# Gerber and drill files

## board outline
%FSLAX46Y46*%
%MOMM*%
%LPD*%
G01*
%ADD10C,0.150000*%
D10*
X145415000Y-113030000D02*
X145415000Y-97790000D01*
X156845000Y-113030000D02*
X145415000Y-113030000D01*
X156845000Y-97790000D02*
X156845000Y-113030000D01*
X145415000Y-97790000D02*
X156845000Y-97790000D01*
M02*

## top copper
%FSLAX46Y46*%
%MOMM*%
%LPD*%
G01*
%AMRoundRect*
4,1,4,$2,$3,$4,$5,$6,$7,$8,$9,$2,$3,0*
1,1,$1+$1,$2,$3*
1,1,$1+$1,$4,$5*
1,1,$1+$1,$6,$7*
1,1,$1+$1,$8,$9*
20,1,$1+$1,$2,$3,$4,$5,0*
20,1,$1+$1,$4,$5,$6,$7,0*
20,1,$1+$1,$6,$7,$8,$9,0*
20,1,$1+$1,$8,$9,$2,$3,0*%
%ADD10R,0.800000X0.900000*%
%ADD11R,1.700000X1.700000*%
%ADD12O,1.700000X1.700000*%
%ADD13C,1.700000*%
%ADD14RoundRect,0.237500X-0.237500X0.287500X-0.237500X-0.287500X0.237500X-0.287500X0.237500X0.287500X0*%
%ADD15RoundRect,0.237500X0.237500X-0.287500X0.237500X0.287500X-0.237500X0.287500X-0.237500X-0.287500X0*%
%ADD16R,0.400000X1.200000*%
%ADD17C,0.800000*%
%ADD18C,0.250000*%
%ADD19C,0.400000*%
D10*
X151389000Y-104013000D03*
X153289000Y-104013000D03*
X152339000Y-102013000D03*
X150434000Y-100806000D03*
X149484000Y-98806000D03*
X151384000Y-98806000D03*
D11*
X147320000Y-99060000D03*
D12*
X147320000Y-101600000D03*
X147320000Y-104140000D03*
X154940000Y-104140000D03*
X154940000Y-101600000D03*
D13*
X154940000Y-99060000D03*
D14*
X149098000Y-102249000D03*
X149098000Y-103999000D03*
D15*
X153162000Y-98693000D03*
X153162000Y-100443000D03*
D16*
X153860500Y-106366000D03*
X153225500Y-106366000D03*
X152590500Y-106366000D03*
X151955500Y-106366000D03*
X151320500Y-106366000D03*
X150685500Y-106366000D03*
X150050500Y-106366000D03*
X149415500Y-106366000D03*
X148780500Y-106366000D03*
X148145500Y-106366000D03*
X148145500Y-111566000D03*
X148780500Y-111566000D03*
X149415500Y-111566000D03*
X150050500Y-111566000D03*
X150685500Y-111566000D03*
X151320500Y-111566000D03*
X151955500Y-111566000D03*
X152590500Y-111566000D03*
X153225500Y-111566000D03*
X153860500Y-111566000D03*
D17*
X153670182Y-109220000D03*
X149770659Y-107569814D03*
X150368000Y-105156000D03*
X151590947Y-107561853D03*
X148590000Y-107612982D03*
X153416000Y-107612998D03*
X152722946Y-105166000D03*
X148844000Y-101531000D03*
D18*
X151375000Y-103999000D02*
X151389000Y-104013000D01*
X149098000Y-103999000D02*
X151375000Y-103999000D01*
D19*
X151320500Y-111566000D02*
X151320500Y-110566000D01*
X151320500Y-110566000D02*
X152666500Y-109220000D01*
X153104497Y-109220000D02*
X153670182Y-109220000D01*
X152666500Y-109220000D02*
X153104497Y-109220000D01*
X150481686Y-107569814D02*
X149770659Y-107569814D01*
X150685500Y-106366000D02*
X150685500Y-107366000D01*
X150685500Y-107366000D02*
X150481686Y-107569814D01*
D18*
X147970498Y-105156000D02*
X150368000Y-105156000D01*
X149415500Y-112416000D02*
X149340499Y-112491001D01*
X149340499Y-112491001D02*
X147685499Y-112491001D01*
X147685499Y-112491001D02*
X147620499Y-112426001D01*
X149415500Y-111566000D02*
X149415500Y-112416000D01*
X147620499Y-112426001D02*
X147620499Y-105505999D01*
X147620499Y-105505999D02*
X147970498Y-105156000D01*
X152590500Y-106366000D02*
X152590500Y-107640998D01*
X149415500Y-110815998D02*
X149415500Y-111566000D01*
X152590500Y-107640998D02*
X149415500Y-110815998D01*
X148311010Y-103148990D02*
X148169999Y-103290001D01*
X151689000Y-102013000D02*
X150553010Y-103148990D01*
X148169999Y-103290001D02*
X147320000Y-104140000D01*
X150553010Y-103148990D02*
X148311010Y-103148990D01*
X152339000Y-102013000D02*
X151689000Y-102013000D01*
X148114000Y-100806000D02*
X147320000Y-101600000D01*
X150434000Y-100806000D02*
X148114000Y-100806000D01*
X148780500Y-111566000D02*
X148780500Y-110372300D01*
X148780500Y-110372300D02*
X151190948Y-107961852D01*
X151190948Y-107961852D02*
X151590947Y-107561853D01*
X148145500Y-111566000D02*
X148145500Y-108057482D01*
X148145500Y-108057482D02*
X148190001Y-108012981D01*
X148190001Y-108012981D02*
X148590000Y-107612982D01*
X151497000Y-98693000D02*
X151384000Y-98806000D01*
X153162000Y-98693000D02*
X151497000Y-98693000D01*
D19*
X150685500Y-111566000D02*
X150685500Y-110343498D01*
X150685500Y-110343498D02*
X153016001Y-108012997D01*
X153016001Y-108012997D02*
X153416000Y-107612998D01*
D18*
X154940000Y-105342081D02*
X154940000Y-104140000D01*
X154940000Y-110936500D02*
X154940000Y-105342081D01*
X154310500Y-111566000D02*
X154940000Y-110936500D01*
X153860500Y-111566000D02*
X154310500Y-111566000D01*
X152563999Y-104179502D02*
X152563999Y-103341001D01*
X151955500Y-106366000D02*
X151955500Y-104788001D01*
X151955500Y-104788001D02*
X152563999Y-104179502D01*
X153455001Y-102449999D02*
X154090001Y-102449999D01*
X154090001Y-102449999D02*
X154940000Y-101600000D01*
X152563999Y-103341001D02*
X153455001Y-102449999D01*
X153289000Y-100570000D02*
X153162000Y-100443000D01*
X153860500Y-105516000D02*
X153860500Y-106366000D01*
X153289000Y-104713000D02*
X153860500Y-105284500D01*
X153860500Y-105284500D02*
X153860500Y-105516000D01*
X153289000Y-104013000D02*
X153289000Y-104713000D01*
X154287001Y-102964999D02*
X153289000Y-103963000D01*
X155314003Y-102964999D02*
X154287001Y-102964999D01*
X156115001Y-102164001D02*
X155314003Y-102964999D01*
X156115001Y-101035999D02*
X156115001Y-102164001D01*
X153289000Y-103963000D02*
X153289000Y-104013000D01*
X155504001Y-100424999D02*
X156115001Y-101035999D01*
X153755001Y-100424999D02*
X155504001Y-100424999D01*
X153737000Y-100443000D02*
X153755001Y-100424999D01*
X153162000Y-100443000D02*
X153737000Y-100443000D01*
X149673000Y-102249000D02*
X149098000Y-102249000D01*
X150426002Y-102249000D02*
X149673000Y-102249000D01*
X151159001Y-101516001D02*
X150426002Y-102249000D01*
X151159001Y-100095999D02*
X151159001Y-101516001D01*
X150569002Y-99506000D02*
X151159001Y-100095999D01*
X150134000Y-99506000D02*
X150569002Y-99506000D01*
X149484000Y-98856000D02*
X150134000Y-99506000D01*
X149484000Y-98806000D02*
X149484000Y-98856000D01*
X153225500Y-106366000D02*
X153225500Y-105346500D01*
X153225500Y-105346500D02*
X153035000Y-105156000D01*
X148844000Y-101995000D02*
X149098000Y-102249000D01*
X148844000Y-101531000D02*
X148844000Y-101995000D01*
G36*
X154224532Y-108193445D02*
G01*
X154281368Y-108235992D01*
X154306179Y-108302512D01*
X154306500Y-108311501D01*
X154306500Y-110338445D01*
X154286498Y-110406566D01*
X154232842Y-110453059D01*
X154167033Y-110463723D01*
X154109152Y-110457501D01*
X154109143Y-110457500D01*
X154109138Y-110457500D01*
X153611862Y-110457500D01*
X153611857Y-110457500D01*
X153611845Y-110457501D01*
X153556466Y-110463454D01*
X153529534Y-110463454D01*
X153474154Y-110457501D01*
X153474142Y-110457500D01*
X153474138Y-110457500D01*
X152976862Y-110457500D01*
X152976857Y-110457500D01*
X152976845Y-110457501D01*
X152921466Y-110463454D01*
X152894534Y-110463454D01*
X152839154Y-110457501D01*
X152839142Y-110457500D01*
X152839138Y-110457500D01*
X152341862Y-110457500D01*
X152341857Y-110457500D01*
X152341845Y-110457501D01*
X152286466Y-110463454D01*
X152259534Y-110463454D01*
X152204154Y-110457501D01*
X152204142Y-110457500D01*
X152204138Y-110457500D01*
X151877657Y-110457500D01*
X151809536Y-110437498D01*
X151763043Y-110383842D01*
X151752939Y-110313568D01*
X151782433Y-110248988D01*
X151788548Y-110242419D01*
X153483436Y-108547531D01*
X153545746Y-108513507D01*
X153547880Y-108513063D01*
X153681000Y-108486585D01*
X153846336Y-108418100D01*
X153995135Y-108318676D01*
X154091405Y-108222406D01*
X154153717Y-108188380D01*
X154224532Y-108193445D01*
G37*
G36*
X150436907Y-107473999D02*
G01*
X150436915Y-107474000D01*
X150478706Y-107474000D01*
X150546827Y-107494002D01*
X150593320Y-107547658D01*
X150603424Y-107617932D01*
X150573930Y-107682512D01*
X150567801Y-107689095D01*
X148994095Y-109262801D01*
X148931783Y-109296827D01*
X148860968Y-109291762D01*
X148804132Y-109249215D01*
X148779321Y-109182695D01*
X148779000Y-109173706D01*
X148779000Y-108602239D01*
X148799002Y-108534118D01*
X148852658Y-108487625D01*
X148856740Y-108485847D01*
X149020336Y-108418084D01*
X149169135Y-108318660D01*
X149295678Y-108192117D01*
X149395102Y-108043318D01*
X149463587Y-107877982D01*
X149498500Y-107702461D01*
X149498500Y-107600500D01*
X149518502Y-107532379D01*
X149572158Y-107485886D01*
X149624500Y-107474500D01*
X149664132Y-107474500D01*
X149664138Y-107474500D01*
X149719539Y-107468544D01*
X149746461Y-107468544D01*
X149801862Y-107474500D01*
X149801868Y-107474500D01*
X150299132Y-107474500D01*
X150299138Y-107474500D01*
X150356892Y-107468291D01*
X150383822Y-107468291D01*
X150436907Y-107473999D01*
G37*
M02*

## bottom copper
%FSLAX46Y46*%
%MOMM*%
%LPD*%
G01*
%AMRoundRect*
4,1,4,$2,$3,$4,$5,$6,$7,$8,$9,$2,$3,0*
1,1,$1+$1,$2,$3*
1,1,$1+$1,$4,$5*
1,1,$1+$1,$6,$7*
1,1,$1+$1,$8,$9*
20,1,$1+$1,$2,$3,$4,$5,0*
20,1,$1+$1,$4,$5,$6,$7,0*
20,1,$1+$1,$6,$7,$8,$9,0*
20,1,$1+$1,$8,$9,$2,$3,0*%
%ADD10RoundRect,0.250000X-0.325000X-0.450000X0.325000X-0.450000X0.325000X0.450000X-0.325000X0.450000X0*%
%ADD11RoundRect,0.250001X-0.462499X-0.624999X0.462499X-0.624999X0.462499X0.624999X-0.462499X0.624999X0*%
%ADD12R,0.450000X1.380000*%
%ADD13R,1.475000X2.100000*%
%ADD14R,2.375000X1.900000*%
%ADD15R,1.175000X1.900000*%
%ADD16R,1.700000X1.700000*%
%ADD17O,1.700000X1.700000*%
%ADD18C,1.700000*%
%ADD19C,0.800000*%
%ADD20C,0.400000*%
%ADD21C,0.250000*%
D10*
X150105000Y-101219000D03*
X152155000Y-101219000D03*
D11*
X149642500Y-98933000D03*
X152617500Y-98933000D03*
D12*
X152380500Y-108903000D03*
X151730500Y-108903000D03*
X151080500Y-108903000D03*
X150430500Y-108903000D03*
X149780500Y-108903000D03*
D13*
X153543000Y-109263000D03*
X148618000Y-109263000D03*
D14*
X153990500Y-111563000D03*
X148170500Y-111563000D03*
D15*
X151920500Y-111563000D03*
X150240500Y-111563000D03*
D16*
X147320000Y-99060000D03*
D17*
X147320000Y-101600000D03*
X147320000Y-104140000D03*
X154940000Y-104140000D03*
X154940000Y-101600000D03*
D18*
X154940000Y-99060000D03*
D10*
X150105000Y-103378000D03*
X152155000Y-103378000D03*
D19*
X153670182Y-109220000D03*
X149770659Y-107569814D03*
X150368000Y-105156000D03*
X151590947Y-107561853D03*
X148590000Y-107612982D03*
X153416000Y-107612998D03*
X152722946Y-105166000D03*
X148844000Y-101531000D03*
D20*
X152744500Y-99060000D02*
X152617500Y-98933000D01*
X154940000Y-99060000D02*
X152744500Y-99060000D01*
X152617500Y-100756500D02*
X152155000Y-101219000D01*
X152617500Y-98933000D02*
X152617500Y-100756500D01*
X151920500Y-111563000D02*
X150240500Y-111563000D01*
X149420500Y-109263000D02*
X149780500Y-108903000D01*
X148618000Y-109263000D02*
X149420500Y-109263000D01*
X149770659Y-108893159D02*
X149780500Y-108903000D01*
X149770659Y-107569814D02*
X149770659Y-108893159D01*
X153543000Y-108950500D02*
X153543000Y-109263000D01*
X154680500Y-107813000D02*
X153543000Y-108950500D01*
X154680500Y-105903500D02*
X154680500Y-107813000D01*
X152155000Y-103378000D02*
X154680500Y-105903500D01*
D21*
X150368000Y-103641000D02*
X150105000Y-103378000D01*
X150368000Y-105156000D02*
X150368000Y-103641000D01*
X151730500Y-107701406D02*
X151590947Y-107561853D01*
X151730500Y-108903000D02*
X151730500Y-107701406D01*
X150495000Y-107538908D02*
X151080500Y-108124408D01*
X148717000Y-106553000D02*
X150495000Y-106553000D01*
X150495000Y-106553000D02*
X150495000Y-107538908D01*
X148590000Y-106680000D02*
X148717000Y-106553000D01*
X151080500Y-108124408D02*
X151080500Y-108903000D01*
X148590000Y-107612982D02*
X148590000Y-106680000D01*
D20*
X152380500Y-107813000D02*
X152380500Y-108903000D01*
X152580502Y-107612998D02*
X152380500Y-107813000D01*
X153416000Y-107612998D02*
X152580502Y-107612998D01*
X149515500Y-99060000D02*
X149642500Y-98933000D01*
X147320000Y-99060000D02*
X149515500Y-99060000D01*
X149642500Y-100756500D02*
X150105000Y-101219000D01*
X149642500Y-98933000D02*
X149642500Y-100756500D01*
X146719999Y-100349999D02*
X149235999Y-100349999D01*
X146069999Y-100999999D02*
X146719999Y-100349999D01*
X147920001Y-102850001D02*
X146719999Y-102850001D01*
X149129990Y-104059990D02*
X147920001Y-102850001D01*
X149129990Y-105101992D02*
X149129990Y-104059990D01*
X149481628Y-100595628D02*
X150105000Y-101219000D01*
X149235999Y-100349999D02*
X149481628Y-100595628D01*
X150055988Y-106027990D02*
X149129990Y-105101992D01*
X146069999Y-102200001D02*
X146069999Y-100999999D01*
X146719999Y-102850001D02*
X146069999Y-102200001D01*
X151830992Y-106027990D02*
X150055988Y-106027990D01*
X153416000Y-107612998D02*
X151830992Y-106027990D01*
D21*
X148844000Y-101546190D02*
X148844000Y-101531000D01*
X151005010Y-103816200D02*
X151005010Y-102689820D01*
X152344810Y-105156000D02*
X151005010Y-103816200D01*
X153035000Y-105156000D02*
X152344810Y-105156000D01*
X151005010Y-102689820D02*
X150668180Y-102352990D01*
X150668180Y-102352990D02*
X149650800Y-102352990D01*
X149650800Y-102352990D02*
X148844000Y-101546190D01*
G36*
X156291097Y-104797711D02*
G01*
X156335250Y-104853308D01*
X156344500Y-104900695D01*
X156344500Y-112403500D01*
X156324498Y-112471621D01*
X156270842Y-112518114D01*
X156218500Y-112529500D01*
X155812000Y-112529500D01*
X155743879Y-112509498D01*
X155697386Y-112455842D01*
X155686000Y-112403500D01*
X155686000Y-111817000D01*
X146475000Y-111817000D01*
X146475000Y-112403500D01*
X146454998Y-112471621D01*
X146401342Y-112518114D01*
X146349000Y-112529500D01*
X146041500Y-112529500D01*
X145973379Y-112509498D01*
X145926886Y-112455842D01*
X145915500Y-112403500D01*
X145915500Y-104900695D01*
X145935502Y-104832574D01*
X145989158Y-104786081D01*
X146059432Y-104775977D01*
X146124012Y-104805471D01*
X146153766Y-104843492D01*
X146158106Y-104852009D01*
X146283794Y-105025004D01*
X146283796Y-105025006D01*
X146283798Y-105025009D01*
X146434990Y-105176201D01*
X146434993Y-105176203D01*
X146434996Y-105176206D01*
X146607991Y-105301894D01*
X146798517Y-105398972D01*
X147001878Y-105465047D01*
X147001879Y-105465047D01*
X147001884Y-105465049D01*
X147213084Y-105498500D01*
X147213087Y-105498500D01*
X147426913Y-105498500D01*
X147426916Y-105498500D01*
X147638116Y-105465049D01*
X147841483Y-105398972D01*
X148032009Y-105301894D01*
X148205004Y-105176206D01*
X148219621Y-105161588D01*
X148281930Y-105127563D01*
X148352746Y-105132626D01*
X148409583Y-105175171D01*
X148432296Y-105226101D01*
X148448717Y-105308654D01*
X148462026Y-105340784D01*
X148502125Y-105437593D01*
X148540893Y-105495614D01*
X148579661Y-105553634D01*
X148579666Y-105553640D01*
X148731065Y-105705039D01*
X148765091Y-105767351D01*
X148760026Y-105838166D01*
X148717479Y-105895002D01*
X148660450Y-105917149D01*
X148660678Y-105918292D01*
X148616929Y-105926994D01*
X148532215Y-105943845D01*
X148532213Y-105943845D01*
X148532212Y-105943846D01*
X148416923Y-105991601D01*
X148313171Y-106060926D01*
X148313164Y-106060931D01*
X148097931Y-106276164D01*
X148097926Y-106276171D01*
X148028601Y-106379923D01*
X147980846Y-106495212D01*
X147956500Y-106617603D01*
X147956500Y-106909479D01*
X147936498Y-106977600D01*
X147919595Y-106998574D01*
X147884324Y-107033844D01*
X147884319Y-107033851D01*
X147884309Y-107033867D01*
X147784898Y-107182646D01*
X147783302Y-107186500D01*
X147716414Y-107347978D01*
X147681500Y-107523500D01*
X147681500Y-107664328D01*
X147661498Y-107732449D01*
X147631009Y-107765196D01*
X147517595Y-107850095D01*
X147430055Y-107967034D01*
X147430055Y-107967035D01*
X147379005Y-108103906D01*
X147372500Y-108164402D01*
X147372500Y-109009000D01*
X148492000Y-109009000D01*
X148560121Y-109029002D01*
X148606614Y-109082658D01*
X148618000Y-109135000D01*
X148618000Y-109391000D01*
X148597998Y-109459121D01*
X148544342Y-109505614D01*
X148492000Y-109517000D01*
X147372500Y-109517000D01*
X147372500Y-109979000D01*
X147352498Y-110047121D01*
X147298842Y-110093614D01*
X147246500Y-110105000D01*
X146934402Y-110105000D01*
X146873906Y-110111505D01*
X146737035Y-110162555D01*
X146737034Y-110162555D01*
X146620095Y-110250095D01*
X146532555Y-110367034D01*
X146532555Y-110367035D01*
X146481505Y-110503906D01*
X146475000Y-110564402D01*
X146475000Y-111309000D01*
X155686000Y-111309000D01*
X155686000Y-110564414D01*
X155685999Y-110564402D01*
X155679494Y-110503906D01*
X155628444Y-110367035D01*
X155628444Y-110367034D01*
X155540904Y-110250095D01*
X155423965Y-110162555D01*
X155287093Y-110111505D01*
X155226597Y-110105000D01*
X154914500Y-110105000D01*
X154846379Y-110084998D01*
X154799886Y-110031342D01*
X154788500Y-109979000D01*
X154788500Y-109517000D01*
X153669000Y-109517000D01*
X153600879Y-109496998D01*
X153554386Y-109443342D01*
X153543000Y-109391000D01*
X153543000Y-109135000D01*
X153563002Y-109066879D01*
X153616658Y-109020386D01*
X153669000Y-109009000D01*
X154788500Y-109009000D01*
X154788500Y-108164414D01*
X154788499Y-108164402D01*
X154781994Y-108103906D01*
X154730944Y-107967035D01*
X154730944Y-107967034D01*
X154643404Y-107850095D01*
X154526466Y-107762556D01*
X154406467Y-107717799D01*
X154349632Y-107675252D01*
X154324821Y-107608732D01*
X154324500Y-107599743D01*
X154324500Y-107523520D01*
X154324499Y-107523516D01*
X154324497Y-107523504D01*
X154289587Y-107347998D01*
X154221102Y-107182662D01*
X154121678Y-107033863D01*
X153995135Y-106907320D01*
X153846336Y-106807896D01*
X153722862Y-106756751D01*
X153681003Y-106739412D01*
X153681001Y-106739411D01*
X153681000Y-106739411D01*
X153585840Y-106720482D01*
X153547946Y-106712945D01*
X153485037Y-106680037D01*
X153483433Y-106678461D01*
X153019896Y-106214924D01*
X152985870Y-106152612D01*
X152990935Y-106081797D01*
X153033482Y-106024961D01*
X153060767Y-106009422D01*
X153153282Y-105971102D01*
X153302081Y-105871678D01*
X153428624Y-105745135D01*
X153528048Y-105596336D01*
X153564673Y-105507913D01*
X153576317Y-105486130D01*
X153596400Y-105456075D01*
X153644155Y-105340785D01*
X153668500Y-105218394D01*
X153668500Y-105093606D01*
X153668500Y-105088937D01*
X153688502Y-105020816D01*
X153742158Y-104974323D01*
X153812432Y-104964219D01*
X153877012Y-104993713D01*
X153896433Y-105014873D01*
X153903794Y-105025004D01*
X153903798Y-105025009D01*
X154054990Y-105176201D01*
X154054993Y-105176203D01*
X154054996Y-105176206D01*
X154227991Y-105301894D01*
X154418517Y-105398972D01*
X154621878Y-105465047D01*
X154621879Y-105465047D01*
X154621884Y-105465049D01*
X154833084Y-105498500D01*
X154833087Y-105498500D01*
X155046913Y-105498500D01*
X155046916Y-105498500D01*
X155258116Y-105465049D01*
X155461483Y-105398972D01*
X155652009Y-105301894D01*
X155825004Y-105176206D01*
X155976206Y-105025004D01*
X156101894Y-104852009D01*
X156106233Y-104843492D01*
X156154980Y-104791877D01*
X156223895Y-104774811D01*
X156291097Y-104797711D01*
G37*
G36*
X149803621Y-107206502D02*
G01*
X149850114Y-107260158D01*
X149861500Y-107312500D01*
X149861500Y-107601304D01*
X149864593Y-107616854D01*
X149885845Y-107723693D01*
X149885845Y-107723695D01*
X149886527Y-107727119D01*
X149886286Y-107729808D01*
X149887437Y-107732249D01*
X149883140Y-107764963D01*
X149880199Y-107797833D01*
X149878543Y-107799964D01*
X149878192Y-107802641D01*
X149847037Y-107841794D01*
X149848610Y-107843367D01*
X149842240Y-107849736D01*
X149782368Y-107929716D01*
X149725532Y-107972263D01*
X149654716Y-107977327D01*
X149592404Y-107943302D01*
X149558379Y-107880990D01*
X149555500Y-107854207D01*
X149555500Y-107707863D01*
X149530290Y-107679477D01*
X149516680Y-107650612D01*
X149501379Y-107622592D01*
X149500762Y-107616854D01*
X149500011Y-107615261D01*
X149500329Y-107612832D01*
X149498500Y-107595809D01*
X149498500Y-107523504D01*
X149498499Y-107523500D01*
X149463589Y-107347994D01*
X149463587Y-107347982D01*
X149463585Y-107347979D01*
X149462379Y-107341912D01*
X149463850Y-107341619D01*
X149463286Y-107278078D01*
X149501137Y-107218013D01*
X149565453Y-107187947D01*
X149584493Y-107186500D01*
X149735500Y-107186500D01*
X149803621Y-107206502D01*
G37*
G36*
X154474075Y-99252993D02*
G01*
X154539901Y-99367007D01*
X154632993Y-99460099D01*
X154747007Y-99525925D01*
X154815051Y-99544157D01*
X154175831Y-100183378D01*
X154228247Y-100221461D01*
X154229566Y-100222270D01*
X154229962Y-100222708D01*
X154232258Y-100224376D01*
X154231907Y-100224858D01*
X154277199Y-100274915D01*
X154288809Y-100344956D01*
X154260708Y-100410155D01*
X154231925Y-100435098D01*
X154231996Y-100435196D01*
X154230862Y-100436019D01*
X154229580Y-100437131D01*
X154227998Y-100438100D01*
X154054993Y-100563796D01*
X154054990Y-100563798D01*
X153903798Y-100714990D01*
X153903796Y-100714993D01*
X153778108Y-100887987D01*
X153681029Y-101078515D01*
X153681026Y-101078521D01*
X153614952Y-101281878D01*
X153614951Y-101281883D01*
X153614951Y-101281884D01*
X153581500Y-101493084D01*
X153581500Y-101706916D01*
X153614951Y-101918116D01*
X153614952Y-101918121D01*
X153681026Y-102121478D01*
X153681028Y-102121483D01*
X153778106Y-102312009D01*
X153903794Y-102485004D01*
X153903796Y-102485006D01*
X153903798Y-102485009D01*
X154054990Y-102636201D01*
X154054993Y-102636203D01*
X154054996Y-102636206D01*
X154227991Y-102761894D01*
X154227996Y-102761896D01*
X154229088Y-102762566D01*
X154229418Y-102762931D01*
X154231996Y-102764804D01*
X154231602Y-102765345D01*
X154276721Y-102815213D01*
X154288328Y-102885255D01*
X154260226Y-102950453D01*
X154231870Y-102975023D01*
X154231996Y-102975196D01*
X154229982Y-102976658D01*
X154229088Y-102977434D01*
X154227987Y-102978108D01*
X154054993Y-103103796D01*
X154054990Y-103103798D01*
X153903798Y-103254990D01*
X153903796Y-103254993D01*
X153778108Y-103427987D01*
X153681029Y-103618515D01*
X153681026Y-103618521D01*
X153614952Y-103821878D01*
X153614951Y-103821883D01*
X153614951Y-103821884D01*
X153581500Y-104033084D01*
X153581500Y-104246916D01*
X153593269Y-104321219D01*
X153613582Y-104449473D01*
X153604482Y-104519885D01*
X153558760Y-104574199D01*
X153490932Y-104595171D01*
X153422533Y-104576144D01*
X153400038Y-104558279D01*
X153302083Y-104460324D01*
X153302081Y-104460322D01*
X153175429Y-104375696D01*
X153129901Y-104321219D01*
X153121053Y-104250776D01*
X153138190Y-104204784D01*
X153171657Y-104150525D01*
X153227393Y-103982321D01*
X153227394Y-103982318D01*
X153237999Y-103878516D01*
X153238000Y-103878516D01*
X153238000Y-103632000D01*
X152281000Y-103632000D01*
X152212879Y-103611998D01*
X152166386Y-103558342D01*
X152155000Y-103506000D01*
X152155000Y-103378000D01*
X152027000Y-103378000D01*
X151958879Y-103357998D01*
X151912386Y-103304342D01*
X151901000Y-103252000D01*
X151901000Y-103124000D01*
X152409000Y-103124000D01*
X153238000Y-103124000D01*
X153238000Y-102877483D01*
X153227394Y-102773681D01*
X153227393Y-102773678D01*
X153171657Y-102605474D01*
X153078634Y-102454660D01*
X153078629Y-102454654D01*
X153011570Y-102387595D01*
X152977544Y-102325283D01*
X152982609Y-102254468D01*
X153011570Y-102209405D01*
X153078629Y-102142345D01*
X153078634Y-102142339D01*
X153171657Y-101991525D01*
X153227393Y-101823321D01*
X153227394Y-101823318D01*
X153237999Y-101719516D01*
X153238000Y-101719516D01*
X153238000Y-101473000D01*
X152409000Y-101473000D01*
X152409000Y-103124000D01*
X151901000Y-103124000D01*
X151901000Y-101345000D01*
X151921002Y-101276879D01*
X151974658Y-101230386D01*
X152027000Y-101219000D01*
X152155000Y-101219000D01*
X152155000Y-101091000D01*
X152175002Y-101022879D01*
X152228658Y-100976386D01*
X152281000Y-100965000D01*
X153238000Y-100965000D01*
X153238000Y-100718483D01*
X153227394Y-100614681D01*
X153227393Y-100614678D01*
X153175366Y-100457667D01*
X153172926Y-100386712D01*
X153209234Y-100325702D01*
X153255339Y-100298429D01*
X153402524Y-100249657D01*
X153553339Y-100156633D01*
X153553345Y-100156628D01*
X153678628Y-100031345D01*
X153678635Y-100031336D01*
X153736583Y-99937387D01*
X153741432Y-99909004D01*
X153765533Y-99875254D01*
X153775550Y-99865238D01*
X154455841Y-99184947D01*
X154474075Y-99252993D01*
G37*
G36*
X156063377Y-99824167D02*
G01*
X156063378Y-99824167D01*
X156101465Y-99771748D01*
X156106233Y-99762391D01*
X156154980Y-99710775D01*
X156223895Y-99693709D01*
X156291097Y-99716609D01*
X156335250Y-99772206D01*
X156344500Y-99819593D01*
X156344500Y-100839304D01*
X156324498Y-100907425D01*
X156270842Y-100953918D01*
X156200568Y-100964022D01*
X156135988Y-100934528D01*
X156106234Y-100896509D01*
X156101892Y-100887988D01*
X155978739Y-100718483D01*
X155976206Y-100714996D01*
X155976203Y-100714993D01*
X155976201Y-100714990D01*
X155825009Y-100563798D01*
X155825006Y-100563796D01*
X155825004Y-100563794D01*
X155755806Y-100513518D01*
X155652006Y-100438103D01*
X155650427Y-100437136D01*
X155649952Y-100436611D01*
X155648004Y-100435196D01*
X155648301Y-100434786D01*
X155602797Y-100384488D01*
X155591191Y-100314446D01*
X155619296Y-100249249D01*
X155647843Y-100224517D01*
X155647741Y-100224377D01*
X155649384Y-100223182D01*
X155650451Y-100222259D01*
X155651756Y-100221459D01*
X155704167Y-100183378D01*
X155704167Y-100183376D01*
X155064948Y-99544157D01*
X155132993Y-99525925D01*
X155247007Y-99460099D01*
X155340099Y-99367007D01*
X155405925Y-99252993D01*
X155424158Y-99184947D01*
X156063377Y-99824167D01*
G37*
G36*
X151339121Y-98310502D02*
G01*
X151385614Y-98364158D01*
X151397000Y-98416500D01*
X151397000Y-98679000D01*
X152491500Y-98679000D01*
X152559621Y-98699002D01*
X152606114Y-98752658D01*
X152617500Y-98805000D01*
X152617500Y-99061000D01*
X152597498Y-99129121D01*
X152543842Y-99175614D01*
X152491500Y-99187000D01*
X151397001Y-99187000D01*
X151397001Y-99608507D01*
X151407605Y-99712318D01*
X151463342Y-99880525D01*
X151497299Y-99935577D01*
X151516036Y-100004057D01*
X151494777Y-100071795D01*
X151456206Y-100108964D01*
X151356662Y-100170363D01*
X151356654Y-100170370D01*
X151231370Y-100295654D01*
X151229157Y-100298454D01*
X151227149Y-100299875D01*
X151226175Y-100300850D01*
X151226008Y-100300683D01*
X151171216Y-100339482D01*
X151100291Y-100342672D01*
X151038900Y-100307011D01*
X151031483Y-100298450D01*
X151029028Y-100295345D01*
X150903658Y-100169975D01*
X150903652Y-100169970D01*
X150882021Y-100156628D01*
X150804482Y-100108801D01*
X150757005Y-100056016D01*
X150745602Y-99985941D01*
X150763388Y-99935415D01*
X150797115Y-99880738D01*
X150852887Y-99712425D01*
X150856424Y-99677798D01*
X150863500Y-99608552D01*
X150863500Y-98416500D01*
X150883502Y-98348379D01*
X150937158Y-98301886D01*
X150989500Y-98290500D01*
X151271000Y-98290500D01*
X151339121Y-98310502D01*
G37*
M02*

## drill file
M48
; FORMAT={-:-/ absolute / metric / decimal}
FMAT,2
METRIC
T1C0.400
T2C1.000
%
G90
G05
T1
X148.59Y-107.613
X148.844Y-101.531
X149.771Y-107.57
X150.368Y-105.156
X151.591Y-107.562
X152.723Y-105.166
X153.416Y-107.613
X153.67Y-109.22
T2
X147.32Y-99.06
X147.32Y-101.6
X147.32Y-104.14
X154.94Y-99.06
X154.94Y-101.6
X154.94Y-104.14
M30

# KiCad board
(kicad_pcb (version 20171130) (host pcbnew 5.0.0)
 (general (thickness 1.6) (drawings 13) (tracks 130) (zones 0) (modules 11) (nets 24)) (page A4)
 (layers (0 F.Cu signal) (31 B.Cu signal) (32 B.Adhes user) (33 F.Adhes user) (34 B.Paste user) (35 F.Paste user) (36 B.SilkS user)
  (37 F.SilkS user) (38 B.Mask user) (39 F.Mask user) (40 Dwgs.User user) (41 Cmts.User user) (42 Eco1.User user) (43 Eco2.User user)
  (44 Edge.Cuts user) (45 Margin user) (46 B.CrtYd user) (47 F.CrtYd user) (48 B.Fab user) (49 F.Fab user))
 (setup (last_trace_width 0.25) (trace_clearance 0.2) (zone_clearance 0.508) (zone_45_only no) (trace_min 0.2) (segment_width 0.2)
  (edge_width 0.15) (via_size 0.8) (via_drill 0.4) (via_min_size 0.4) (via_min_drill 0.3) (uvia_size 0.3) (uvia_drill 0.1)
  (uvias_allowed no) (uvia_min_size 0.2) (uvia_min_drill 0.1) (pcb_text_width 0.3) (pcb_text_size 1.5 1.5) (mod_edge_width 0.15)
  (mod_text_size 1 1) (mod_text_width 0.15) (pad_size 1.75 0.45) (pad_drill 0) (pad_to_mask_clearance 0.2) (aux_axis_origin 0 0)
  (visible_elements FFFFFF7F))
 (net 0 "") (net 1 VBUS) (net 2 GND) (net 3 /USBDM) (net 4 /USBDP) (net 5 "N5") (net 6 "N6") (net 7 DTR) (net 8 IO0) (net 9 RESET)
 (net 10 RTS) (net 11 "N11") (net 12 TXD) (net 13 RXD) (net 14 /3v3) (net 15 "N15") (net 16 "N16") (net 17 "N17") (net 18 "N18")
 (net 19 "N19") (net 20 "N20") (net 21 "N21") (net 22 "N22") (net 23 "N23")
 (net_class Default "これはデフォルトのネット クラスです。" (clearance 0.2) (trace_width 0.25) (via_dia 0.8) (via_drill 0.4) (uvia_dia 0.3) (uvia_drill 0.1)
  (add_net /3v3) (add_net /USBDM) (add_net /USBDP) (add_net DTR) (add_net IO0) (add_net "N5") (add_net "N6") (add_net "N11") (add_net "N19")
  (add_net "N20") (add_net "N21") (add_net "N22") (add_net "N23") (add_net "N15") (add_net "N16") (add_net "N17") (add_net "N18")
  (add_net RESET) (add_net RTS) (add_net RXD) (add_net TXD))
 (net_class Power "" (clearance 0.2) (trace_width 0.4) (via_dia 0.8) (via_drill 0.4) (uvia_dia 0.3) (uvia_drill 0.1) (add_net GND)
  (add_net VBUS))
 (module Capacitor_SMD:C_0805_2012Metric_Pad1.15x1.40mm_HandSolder (layer B.Cu) (at 151.13 101.219)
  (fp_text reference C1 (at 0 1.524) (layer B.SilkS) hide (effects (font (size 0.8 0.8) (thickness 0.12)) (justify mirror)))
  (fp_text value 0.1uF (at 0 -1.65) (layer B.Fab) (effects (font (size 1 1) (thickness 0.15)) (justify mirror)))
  (pad 1 smd roundrect (at -1.025 0) (size 1.15 1.4) (layers B.Cu B.Paste B.Mask) (roundrect_rratio 0.217391) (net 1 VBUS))
  (pad 2 smd roundrect (at 1.025 0) (size 1.15 1.4) (layers B.Cu B.Paste B.Mask) (roundrect_rratio 0.217391) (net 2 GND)))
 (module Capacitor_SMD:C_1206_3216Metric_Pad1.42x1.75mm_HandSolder (layer B.Cu) (at 151.13 98.933)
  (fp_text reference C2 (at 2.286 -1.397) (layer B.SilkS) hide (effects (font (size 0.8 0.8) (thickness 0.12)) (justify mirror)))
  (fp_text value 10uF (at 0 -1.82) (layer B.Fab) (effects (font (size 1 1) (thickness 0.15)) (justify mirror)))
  (pad 1 smd roundrect (at -1.4875 0) (size 1.425 1.75) (layers B.Cu B.Paste B.Mask) (roundrect_rratio 0.175439) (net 1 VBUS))
  (pad 2 smd roundrect (at 1.4875 0) (size 1.425 1.75) (layers B.Cu B.Paste B.Mask) (roundrect_rratio 0.175439) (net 2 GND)))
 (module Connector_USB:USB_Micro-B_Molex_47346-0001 (layer B.Cu) (at 151.0805 110.363 180)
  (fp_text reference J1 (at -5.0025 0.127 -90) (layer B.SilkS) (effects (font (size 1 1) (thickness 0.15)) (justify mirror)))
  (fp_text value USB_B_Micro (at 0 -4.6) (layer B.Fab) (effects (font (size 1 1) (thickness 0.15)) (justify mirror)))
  (pad 1 smd rect (at -1.3 1.46 180) (size 0.45 1.38) (layers B.Cu B.Paste B.Mask) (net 1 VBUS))
  (pad 2 smd rect (at -0.65 1.46 180) (size 0.45 1.38) (layers B.Cu B.Paste B.Mask) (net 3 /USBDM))
  (pad 3 smd rect (at 0 1.46 180) (size 0.45 1.38) (layers B.Cu B.Paste B.Mask) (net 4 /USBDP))
  (pad 4 smd rect (at 0.65 1.46 180) (size 0.45 1.38) (layers B.Cu B.Paste B.Mask) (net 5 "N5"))
  (pad 5 smd rect (at 1.3 1.46 180) (size 0.45 1.38) (layers B.Cu B.Paste B.Mask) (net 2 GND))
  (pad 6 smd rect (at -2.4625 1.1 180) (size 1.475 2.1) (layers B.Cu B.Paste B.Mask) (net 2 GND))
  (pad 6 smd rect (at 2.4625 1.1 180) (size 1.475 2.1) (layers B.Cu B.Paste B.Mask) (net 2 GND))
  (pad 6 smd rect (at -2.91 -1.2 180) (size 2.375 1.9) (layers B.Cu B.Paste B.Mask) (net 2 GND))
  (pad 6 smd rect (at 2.91 -1.2 180) (size 2.375 1.9) (layers B.Cu B.Paste B.Mask) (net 2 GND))
  (pad 6 smd rect (at -0.84 -1.2 180) (size 1.175 1.9) (layers B.Cu B.Paste B.Mask) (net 2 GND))
  (pad 6 smd rect (at 0.84 -1.2 180) (size 1.175 1.9) (layers B.Cu B.Paste B.Mask) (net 2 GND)))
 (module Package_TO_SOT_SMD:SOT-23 (layer F.Cu) (at 152.339 103.013 90)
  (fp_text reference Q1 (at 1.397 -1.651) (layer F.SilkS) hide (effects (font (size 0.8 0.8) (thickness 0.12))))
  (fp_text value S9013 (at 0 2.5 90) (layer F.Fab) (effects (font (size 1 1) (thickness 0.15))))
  (pad 1 smd rect (at -1 -0.95 90) (size 0.9 0.8) (layers F.Cu F.Paste F.Mask) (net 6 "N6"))
  (pad 2 smd rect (at -1 0.95 90) (size 0.9 0.8) (layers F.Cu F.Paste F.Mask) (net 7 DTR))
  (pad 3 smd rect (at 1 0 90) (size 0.9 0.8) (layers F.Cu F.Paste F.Mask) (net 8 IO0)))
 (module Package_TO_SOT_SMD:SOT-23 (layer F.Cu) (at 150.434 99.806 270)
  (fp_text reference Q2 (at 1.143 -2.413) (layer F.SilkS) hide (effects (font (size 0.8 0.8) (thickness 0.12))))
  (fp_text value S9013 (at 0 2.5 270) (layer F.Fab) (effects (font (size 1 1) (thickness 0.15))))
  (pad 3 smd rect (at 1 0 270) (size 0.9 0.8) (layers F.Cu F.Paste F.Mask) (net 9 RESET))
  (pad 2 smd rect (at -1 0.95 270) (size 0.9 0.8) (layers F.Cu F.Paste F.Mask) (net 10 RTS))
  (pad 1 smd rect (at -1 -0.95 270) (size 0.9 0.8) (layers F.Cu F.Paste F.Mask) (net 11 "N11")))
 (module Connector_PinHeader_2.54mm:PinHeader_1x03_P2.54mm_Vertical (layer B.Cu) (at 147.32 99.06 180)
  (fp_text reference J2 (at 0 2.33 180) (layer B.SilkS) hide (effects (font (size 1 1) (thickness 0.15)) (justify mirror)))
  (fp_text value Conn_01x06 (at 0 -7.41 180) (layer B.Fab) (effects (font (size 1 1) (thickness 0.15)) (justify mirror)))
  (pad 1 thru_hole rect (at 0 0 180) (size 1.7 1.7) (drill 1) (layers *.Cu *.Mask) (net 1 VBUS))
  (pad 2 thru_hole oval (at 0 -2.54 180) (size 1.7 1.7) (drill 1) (layers *.Cu *.Mask) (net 9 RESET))
  (pad 3 thru_hole oval (at 0 -5.08 180) (size 1.7 1.7) (drill 1) (layers *.Cu *.Mask) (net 8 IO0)))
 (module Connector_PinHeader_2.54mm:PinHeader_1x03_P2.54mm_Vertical (layer B.Cu) (at 154.94 99.06 180)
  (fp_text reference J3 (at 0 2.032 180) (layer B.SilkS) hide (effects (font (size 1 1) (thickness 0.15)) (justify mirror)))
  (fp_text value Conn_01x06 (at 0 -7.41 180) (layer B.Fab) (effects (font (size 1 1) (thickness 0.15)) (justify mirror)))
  (pad 3 thru_hole oval (at 0 -5.08 180) (size 1.7 1.7) (drill 1) (layers *.Cu *.Mask) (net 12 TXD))
  (pad 2 thru_hole oval (at 0 -2.54 180) (size 1.7 1.7) (drill 1) (layers *.Cu *.Mask) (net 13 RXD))
  (pad 1 thru_hole circle (at 0 0 180) (size 1.7 1.7) (drill 1) (layers *.Cu *.Mask) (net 2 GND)))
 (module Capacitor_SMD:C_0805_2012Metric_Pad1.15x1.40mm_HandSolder (layer B.Cu) (at 151.13 103.378)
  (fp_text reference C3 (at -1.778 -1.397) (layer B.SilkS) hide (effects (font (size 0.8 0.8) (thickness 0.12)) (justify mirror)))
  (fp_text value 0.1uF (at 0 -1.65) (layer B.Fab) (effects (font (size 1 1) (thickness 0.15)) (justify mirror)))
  (pad 1 smd roundrect (at -1.025 0) (size 1.15 1.4) (layers B.Cu B.Paste B.Mask) (roundrect_rratio 0.217391) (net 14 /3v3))
  (pad 2 smd roundrect (at 1.025 0) (size 1.15 1.4) (layers B.Cu B.Paste B.Mask) (roundrect_rratio 0.217391) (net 2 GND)))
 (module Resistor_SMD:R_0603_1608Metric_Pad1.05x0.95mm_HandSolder (layer F.Cu) (at 149.098 103.124 270)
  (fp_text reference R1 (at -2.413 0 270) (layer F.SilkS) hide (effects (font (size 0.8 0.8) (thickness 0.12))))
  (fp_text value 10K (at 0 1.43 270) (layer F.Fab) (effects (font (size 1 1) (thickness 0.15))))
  (pad 1 smd roundrect (at -0.875 0 270) (size 1.05 0.95) (layers F.Cu F.Paste F.Mask) (roundrect_rratio 0.25) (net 10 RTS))
  (pad 2 smd roundrect (at 0.875 0 270) (size 1.05 0.95) (layers F.Cu F.Paste F.Mask) (roundrect_rratio 0.25) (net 6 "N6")))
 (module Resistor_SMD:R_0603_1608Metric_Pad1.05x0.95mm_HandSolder (layer F.Cu) (at 153.162 99.568 90)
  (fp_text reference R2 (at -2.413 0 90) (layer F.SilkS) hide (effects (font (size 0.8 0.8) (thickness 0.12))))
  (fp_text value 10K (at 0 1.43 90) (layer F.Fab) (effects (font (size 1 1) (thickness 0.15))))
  (pad 2 smd roundrect (at 0.875 0 90) (size 1.05 0.95) (layers F.Cu F.Paste F.Mask) (roundrect_rratio 0.25) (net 11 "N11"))
  (pad 1 smd roundrect (at -0.875 0 90) (size 1.05 0.95) (layers F.Cu F.Paste F.Mask) (roundrect_rratio 0.25) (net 7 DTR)))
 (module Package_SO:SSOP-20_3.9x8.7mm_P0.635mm (layer F.Cu) (at 151.003 108.966 270)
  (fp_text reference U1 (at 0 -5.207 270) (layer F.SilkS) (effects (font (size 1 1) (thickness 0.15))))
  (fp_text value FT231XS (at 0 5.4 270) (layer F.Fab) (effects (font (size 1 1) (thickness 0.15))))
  (pad 1 smd rect (at -2.6 -2.8575 270) (size 1.2 0.4) (layers F.Cu F.Paste F.Mask) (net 7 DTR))
  (pad 2 smd rect (at -2.6 -2.2225 270) (size 1.2 0.4) (layers F.Cu F.Paste F.Mask) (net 10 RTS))
  (pad 3 smd rect (at -2.6 -1.5875 270) (size 1.2 0.4) (layers F.Cu F.Paste F.Mask) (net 14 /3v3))
  (pad 4 smd rect (at -2.6 -0.9525 270) (size 1.2 0.4) (layers F.Cu F.Paste F.Mask) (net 13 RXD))
  (pad 5 smd rect (at -2.6 -0.3175 270) (size 1.2 0.4) (layers F.Cu F.Paste F.Mask) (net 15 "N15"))
  (pad 6 smd rect (at -2.6 0.3175 270) (size 1.2 0.4) (layers F.Cu F.Paste F.Mask) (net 2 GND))
  (pad 7 smd rect (at -2.6 0.9525 270) (size 1.2 0.4) (layers F.Cu F.Paste F.Mask) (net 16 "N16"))
  (pad 8 smd rect (at -2.6 1.5875 270) (size 1.2 0.4) (layers F.Cu F.Paste F.Mask) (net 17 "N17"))
  (pad 9 smd rect (at -2.6 2.2225 270) (size 1.2 0.4) (layers F.Cu F.Paste F.Mask) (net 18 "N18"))
  (pad 10 smd rect (at -2.6 2.8575 270) (size 1.2 0.4) (layers F.Cu F.Paste F.Mask) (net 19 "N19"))
  (pad 11 smd rect (at 2.6 2.8575 270) (size 1.2 0.4) (layers F.Cu F.Paste F.Mask) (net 4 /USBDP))
  (pad 12 smd rect (at 2.6 2.2225 270) (size 1.2 0.4) (layers F.Cu F.Paste F.Mask) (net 3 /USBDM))
  (pad 13 smd rect (at 2.6 1.5875 270) (size 1.2 0.4) (layers F.Cu F.Paste F.Mask) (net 14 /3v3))
  (pad 14 smd rect (at 2.6 0.9525 270) (size 1.2 0.4) (layers F.Cu F.Paste F.Mask) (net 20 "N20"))
  (pad 15 smd rect (at 2.6 0.3175 270) (size 1.2 0.4) (layers F.Cu F.Paste F.Mask) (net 1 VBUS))
  (pad 16 smd rect (at 2.6 -0.3175 270) (size 1.2 0.4) (layers F.Cu F.Paste F.Mask) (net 2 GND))
  (pad 17 smd rect (at 2.6 -0.9525 270) (size 1.2 0.4) (layers F.Cu F.Paste F.Mask) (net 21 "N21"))
  (pad 18 smd rect (at 2.6 -1.5875 270) (size 1.2 0.4) (layers F.Cu F.Paste F.Mask) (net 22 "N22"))
  (pad 19 smd rect (at 2.6 -2.2225 270) (size 1.2 0.4) (layers F.Cu F.Paste F.Mask) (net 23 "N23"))
  (pad 20 smd rect (at 2.6 -2.8575 270) (size 1.2 0.4) (layers F.Cu F.Paste F.Mask) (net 12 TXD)))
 (gr_line (start 145.415 113.03) (end 145.415 97.79) (layer Edge.Cuts) (width 0.15))
 (gr_line (start 156.845 113.03) (end 145.415 113.03) (layer Edge.Cuts) (width 0.15))
 (gr_line (start 156.845 97.79) (end 156.845 113.03) (layer Edge.Cuts) (width 0.15))
 (gr_line (start 145.415 97.79) (end 156.845 97.79) (layer Edge.Cuts) (width 0.15))
 (segment (start 151.375 103.999) (end 151.389 104.013) (width 0.25) (layer F.Cu) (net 6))
 (segment (start 149.098 103.999) (end 151.375 103.999) (width 0.25) (layer F.Cu) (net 6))
 (segment (start 152.7445 99.06) (end 152.6175 98.933) (width 0.4) (layer B.Cu) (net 2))
 (segment (start 154.94 99.06) (end 152.7445 99.06) (width 0.4) (layer B.Cu) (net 2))
 (segment (start 152.6175 100.7565) (end 152.155 101.219) (width 0.4) (layer B.Cu) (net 2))
 (segment (start 152.6175 98.933) (end 152.6175 100.7565) (width 0.4) (layer B.Cu) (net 2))
 (segment (start 151.9205 111.563) (end 150.2405 111.563) (width 0.4) (layer B.Cu) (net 2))
 (segment (start 149.4205 109.263) (end 149.7805 108.903) (width 0.4) (layer B.Cu) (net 2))
 (segment (start 148.618 109.263) (end 149.4205 109.263) (width 0.4) (layer B.Cu) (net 2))
 (via (at 153.670182 109.22) (size 0.8) (drill 0.4) (layers F.Cu B.Cu) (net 2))
 (segment (start 151.3205 111.566) (end 151.3205 110.566) (width 0.4) (layer F.Cu) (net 2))
 (segment (start 151.3205 110.566) (end 152.6665 109.22) (width 0.4) (layer F.Cu) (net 2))
 (segment (start 153.104497 109.22) (end 153.670182 109.22) (width 0.4) (layer F.Cu) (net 2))
 (segment (start 152.6665 109.22) (end 153.104497 109.22) (width 0.4) (layer F.Cu) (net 2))
 (segment (start 150.481686 107.569814) (end 149.770659 107.569814) (width 0.4) (layer F.Cu) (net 2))
 (segment (start 150.6855 106.366) (end 150.6855 107.366) (width 0.4) (layer F.Cu) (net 2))
 (via (at 149.770659 107.569814) (size 0.8) (drill 0.4) (layers F.Cu B.Cu) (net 2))
 (segment (start 150.6855 107.366) (end 150.481686 107.569814) (width 0.4) (layer F.Cu) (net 2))
 (segment (start 149.770659 108.893159) (end 149.7805 108.903) (width 0.4) (layer B.Cu) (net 2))
 (segment (start 149.770659 107.569814) (end 149.770659 108.893159) (width 0.4) (layer B.Cu) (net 2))
 (segment (start 153.543 108.9505) (end 153.543 109.263) (width 0.4) (layer B.Cu) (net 2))
 (segment (start 154.6805 107.813) (end 153.543 108.9505) (width 0.4) (layer B.Cu) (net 2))
 (segment (start 154.6805 105.9035) (end 154.6805 107.813) (width 0.4) (layer B.Cu) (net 2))
 (segment (start 152.155 103.378) (end 154.6805 105.9035) (width 0.4) (layer B.Cu) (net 2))
 (via (at 150.368 105.156) (size 0.8) (drill 0.4) (layers F.Cu B.Cu) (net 14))
 (segment (start 147.970498 105.156) (end 150.368 105.156) (width 0.25) (layer F.Cu) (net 14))
 (segment (start 149.4155 112.416) (end 149.340499 112.491001) (width 0.25) (layer F.Cu) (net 14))
 (segment (start 149.340499 112.491001) (end 147.685499 112.491001) (width 0.25) (layer F.Cu) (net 14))
 (segment (start 147.685499 112.491001) (end 147.620499 112.426001) (width 0.25) (layer F.Cu) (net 14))
 (segment (start 149.4155 111.566) (end 149.4155 112.416) (width 0.25) (layer F.Cu) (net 14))
 (segment (start 147.620499 112.426001) (end 147.620499 105.505999) (width 0.25) (layer F.Cu) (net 14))
 (segment (start 147.620499 105.505999) (end 147.970498 105.156) (width 0.25) (layer F.Cu) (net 14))
 (segment (start 150.368 103.641) (end 150.105 103.378) (width 0.25) (layer B.Cu) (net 14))
 (segment (start 150.368 105.156) (end 150.368 103.641) (width 0.25) (layer B.Cu) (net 14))
 (segment (start 152.5905 106.366) (end 152.5905 107.640998) (width 0.25) (layer F.Cu) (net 14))
 (segment (start 149.4155 110.815998) (end 149.4155 111.566) (width 0.25) (layer F.Cu) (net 14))
 (segment (start 152.5905 107.640998) (end 149.4155 110.815998) (width 0.25) (layer F.Cu) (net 14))
 (segment (start 148.31101 103.14899) (end 148.169999 103.290001) (width 0.25) (layer F.Cu) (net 8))
 (segment (start 151.689 102.013) (end 150.55301 103.14899) (width 0.25) (layer F.Cu) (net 8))
 (segment (start 148.169999 103.290001) (end 147.32 104.14) (width 0.25) (layer F.Cu) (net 8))
 (segment (start 150.55301 103.14899) (end 148.31101 103.14899) (width 0.25) (layer F.Cu) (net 8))
 (segment (start 152.339 102.013) (end 151.689 102.013) (width 0.25) (layer F.Cu) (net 8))
 (segment (start 148.114 100.806) (end 147.32 101.6) (width 0.25) (layer F.Cu) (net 9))
 (segment (start 150.434 100.806) (end 148.114 100.806) (width 0.25) (layer F.Cu) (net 9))
 (segment (start 151.7305 107.701406) (end 151.590947 107.561853) (width 0.25) (layer B.Cu) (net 3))
 (segment (start 148.7805 111.566) (end 148.7805 110.3723) (width 0.25) (layer F.Cu) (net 3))
 (segment (start 148.7805 110.3723) (end 151.190948 107.961852) (width 0.25) (layer F.Cu) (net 3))
 (via (at 151.590947 107.561853) (size 0.8) (drill 0.4) (layers F.Cu B.Cu) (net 3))
 (segment (start 151.190948 107.961852) (end 151.590947 107.561853) (width 0.25) (layer F.Cu) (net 3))
 (segment (start 151.7305 108.903) (end 151.7305 107.701406) (width 0.25) (layer B.Cu) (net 3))
 (via (at 148.59 107.612982) (size 0.8) (drill 0.4) (layers F.Cu B.Cu) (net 4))
 (segment (start 148.1455 111.566) (end 148.1455 108.057482) (width 0.25) (layer F.Cu) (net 4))
 (segment (start 148.1455 108.057482) (end 148.190001 108.012981) (width 0.25) (layer F.Cu) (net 4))
 (segment (start 148.190001 108.012981) (end 148.59 107.612982) (width 0.25) (layer F.Cu) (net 4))
 (segment (start 150.495 107.538908) (end 151.0805 108.124408) (width 0.25) (layer B.Cu) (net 4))
 (segment (start 148.717 106.553) (end 150.495 106.553) (width 0.25) (layer B.Cu) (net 4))
 (segment (start 150.495 106.553) (end 150.495 107.538908) (width 0.25) (layer B.Cu) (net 4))
 (segment (start 148.59 106.68) (end 148.717 106.553) (width 0.25) (layer B.Cu) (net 4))
 (segment (start 151.0805 108.124408) (end 151.0805 108.903) (width 0.25) (layer B.Cu) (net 4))
 (segment (start 148.59 107.612982) (end 148.59 106.68) (width 0.25) (layer B.Cu) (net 4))
 (segment (start 151.497 98.693) (end 151.384 98.806) (width 0.25) (layer F.Cu) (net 11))
 (segment (start 153.162 98.693) (end 151.497 98.693) (width 0.25) (layer F.Cu) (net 11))
 (via (at 153.416 107.612998) (size 0.8) (drill 0.4) (layers F.Cu B.Cu) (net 1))
 (segment (start 152.3805 107.813) (end 152.3805 108.903) (width 0.4) (layer B.Cu) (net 1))
 (segment (start 152.580502 107.612998) (end 152.3805 107.813) (width 0.4) (layer B.Cu) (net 1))
 (segment (start 153.416 107.612998) (end 152.580502 107.612998) (width 0.4) (layer B.Cu) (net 1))
 (segment (start 149.5155 99.06) (end 149.6425 98.933) (width 0.4) (layer B.Cu) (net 1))
 (segment (start 147.32 99.06) (end 149.5155 99.06) (width 0.4) (layer B.Cu) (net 1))
 (segment (start 149.6425 100.7565) (end 150.105 101.219) (width 0.4) (layer B.Cu) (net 1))
 (segment (start 149.6425 98.933) (end 149.6425 100.7565) (width 0.4) (layer B.Cu) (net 1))
 (segment (start 150.6855 111.566) (end 150.6855 110.343498) (width 0.4) (layer F.Cu) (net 1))
 (segment (start 150.6855 110.343498) (end 153.016001 108.012997) (width 0.4) (layer F.Cu) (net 1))
 (segment (start 153.016001 108.012997) (end 153.416 107.612998) (width 0.4) (layer F.Cu) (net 1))
 (segment (start 146.719999 100.349999) (end 149.235999 100.349999) (width 0.4) (layer B.Cu) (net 1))
 (segment (start 146.069999 100.999999) (end 146.719999 100.349999) (width 0.4) (layer B.Cu) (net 1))
 (segment (start 147.920001 102.850001) (end 146.719999 102.850001) (width 0.4) (layer B.Cu) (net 1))
 (segment (start 149.12999 104.05999) (end 147.920001 102.850001) (width 0.4) (layer B.Cu) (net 1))
 (segment (start 149.12999 105.101992) (end 149.12999 104.05999) (width 0.4) (layer B.Cu) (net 1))
 (segment (start 149.481628 100.595628) (end 150.105 101.219) (width 0.4) (layer B.Cu) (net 1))
 (segment (start 149.235999 100.349999) (end 149.481628 100.595628) (width 0.4) (layer B.Cu) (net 1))
 (segment (start 150.055988 106.02799) (end 149.12999 105.101992) (width 0.4) (layer B.Cu) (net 1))
 (segment (start 146.069999 102.200001) (end 146.069999 100.999999) (width 0.4) (layer B.Cu) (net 1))
 (segment (start 146.719999 102.850001) (end 146.069999 102.200001) (width 0.4) (layer B.Cu) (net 1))
 (segment (start 151.830992 106.02799) (end 150.055988 106.02799) (width 0.4) (layer B.Cu) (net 1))
 (segment (start 153.416 107.612998) (end 151.830992 106.02799) (width 0.4) (layer B.Cu) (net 1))
 (segment (start 154.94 105.342081) (end 154.94 104.14) (width 0.25) (layer F.Cu) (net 12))
 (segment (start 154.94 110.9365) (end 154.94 105.342081) (width 0.25) (layer F.Cu) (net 12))
 (segment (start 154.3105 111.566) (end 154.94 110.9365) (width 0.25) (layer F.Cu) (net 12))
 (segment (start 153.8605 111.566) (end 154.3105 111.566) (width 0.25) (layer F.Cu) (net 12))
 (segment (start 152.563999 104.179502) (end 152.563999 103.341001) (width 0.25) (layer F.Cu) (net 13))
 (segment (start 151.9555 106.366) (end 151.9555 104.788001) (width 0.25) (layer F.Cu) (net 13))
 (segment (start 151.9555 104.788001) (end 152.563999 104.179502) (width 0.25) (layer F.Cu) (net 13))
 (segment (start 153.455001 102.449999) (end 154.090001 102.449999) (width 0.25) (layer F.Cu) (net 13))
 (segment (start 154.090001 102.449999) (end 154.94 101.6) (width 0.25) (layer F.Cu) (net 13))
 (segment (start 152.563999 103.341001) (end 153.455001 102.449999) (width 0.25) (layer F.Cu) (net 13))
 (segment (start 153.289 100.57) (end 153.162 100.443) (width 0.25) (layer F.Cu) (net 7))
 (segment (start 153.8605 105.516) (end 153.8605 106.366) (width 0.25) (layer F.Cu) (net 7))
 (segment (start 153.289 104.713) (end 153.8605 105.2845) (width 0.25) (layer F.Cu) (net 7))
 (segment (start 153.8605 105.2845) (end 153.8605 105.516) (width 0.25) (layer F.Cu) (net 7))
 (segment (start 153.289 104.013) (end 153.289 104.713) (width 0.25) (layer F.Cu) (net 7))
 (segment (start 154.287001 102.964999) (end 153.289 103.963) (width 0.25) (layer F.Cu) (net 7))
 (segment (start 155.314003 102.964999) (end 154.287001 102.964999) (width 0.25) (layer F.Cu) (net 7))
 (segment (start 156.115001 102.164001) (end 155.314003 102.964999) (width 0.25) (layer F.Cu) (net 7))
 (segment (start 156.115001 101.035999) (end 156.115001 102.164001) (width 0.25) (layer F.Cu) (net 7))
 (segment (start 153.289 103.963) (end 153.289 104.013) (width 0.25) (layer F.Cu) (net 7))
 (segment (start 155.504001 100.424999) (end 156.115001 101.035999) (width 0.25) (layer F.Cu) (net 7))
 (segment (start 153.755001 100.424999) (end 155.504001 100.424999) (width 0.25) (layer F.Cu) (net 7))
 (segment (start 153.737 100.443) (end 153.755001 100.424999) (width 0.25) (layer F.Cu) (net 7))
 (segment (start 153.162 100.443) (end 153.737 100.443) (width 0.25) (layer F.Cu) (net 7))
 (segment (start 149.673 102.249) (end 149.098 102.249) (width 0.25) (layer F.Cu) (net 10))
 (segment (start 150.426002 102.249) (end 149.673 102.249) (width 0.25) (layer F.Cu) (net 10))
 (segment (start 151.159001 101.516001) (end 150.426002 102.249) (width 0.25) (layer F.Cu) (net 10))
 (segment (start 151.159001 100.095999) (end 151.159001 101.516001) (width 0.25) (layer F.Cu) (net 10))
 (segment (start 150.569002 99.506) (end 151.159001 100.095999) (width 0.25) (layer F.Cu) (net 10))
 (segment (start 150.134 99.506) (end 150.569002 99.506) (width 0.25) (layer F.Cu) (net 10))
 (segment (start 149.484 98.856) (end 150.134 99.506) (width 0.25) (layer F.Cu) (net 10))
 (segment (start 149.484 98.806) (end 149.484 98.856) (width 0.25) (layer F.Cu) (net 10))
 (via (at 152.722946 105.166) (size 0.8) (drill 0.4) (layers F.Cu B.Cu) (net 10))
 (segment (start 153.2255 106.366) (end 153.2255 105.3465) (width 0.25) (layer F.Cu) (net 10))
 (segment (start 153.2255 105.3465) (end 153.035 105.156) (width 0.25) (layer F.Cu) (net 10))
 (via (at 148.844 101.531) (size 0.8) (drill 0.4) (layers F.Cu B.Cu) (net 10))
 (segment (start 148.844 101.54619) (end 148.844 101.531) (width 0.25) (layer B.Cu) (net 10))
 (segment (start 151.00501 103.8162) (end 151.00501 102.68982) (width 0.25) (layer B.Cu) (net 10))
 (segment (start 152.34481 105.156) (end 151.00501 103.8162) (width 0.25) (layer B.Cu) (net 10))
 (segment (start 153.035 105.156) (end 152.34481 105.156) (width 0.25) (layer B.Cu) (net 10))
 (segment (start 151.00501 102.68982) (end 150.66818 102.35299) (width 0.25) (layer B.Cu) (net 10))
 (segment (start 150.66818 102.35299) (end 149.6508 102.35299) (width 0.25) (layer B.Cu) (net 10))
 (segment (start 149.6508 102.35299) (end 148.844 101.54619) (width 0.25) (layer B.Cu) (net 10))
 (segment (start 148.844 101.995) (end 149.098 102.249) (width 0.25) (layer F.Cu) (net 10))
 (segment (start 148.844 101.531) (end 148.844 101.995) (width 0.25) (layer F.Cu) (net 10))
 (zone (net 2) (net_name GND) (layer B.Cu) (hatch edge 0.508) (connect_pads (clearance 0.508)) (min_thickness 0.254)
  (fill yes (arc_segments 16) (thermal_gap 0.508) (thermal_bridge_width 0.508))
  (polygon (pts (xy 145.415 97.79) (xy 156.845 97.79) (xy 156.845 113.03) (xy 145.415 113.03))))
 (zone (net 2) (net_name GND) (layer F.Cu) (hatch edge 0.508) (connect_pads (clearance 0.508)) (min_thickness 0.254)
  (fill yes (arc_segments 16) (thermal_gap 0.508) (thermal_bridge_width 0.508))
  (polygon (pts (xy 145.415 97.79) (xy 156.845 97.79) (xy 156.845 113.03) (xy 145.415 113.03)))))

